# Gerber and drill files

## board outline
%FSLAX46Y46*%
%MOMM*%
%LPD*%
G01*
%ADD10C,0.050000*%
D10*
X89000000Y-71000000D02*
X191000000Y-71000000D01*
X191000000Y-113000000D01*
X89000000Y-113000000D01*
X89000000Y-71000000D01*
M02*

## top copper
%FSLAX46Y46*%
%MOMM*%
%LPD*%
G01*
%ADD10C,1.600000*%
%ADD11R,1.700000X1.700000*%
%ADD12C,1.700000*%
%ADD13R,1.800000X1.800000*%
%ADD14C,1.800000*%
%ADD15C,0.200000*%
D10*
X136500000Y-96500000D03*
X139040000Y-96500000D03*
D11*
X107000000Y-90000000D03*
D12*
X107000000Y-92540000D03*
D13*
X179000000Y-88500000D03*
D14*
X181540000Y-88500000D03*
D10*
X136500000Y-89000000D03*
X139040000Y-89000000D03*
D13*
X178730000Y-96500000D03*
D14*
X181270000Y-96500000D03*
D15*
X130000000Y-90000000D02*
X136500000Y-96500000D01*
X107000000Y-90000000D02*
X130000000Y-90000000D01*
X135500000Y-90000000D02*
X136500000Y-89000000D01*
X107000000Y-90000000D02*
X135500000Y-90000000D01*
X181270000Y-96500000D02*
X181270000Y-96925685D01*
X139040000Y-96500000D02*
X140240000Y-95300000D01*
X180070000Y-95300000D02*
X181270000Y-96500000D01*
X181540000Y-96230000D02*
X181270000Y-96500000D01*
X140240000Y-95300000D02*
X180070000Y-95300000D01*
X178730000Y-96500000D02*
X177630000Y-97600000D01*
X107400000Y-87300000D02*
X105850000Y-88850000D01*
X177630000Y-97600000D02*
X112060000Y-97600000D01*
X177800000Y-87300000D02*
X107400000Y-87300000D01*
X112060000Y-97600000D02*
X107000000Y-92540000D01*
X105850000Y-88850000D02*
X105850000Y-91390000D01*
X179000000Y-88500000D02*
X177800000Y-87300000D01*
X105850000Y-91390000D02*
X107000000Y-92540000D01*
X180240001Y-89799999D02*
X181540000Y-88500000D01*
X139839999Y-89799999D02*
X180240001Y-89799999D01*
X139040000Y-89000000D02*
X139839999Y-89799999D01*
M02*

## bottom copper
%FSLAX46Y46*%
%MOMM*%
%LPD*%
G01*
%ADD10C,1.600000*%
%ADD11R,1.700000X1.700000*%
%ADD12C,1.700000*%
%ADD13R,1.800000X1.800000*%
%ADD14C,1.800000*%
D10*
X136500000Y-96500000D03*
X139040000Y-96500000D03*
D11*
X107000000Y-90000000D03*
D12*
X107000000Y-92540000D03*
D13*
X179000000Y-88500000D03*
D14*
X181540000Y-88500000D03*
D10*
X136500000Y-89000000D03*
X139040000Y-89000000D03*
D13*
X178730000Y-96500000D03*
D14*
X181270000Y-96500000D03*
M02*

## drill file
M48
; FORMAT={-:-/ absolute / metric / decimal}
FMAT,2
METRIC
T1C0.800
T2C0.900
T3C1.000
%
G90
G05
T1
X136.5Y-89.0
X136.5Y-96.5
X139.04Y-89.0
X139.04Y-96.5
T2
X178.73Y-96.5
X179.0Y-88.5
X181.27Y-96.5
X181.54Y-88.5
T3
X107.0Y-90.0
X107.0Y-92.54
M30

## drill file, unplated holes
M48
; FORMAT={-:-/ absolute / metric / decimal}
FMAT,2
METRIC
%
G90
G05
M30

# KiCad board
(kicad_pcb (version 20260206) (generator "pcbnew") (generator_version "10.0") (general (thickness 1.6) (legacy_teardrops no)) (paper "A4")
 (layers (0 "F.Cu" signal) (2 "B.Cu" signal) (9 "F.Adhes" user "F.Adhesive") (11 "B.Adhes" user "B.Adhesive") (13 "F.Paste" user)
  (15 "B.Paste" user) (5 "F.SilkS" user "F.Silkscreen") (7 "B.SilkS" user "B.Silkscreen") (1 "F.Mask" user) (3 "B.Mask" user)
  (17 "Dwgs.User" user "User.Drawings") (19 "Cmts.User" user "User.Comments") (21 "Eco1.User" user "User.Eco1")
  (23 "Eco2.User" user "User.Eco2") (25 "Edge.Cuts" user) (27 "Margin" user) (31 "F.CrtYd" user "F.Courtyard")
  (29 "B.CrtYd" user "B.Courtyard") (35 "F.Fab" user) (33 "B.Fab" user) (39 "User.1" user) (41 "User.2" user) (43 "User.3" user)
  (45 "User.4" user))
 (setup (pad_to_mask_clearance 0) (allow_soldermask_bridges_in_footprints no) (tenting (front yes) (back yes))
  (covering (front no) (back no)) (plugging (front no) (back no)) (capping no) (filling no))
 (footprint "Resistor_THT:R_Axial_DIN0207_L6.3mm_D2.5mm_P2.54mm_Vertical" (layer "F.Cu") (at 136.5 96.5)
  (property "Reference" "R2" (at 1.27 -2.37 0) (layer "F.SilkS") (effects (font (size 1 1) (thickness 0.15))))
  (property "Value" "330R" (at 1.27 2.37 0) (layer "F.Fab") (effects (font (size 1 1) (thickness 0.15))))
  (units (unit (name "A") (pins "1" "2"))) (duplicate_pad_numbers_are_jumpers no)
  (pad "1" thru_hole circle (at 0 0) (size 1.6 1.6) (drill 0.8) (layers "*.Cu" "*.Mask") (remove_unused_layers no) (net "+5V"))
  (pad "2" thru_hole circle (at 2.54 0) (size 1.6 1.6) (drill 0.8) (layers "*.Cu" "*.Mask") (remove_unused_layers no) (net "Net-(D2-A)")))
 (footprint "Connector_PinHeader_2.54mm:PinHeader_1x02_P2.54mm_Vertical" (layer "F.Cu") (at 107 90)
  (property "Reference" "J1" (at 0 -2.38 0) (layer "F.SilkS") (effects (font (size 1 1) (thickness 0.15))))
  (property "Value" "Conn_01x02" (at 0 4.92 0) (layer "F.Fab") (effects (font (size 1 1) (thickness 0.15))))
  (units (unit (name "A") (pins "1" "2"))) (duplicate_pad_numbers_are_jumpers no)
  (pad "1" thru_hole rect (at 0 0) (size 1.7 1.7) (drill 1) (layers "*.Cu" "*.Mask") (remove_unused_layers no) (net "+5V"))
  (pad "2" thru_hole circle (at 0 2.54) (size 1.7 1.7) (drill 1) (layers "*.Cu" "*.Mask") (remove_unused_layers no) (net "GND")))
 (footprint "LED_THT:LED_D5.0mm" (layer "F.Cu") (at 179 88.5)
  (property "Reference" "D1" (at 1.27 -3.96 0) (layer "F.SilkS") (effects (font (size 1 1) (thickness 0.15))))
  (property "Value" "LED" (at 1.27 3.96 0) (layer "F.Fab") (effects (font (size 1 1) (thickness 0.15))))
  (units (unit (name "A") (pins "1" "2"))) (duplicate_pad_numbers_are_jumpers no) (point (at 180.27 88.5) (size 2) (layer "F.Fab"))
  (pad "1" thru_hole rect (at 0 0) (size 1.8 1.8) (drill 0.9) (layers "*.Cu" "*.Mask") (remove_unused_layers no) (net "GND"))
  (pad "2" thru_hole circle (at 2.54 0) (size 1.8 1.8) (drill 0.9) (layers "*.Cu" "*.Mask") (remove_unused_layers no) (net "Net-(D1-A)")))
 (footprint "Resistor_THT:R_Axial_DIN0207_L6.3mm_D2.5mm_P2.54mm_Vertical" (layer "F.Cu") (at 136.5 89)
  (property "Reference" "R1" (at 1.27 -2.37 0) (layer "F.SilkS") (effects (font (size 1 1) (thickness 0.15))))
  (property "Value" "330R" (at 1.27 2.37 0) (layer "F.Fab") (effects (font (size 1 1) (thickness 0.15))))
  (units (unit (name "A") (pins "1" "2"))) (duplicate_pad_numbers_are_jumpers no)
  (pad "1" thru_hole circle (at 0 0) (size 1.6 1.6) (drill 0.8) (layers "*.Cu" "*.Mask") (remove_unused_layers no) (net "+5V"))
  (pad "2" thru_hole circle (at 2.54 0) (size 1.6 1.6) (drill 0.8) (layers "*.Cu" "*.Mask") (remove_unused_layers no) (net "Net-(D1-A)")))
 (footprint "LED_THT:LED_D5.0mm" (layer "F.Cu") (at 178.73 96.5)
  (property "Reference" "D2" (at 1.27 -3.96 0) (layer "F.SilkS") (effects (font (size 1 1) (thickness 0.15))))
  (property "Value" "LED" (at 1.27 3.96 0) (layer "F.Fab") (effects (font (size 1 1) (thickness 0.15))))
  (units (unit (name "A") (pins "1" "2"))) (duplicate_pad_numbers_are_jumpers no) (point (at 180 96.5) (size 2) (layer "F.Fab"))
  (pad "1" thru_hole rect (at 0 0) (size 1.8 1.8) (drill 0.9) (layers "*.Cu" "*.Mask") (remove_unused_layers no) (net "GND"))
  (pad "2" thru_hole circle (at 2.54 0) (size 1.8 1.8) (drill 0.9) (layers "*.Cu" "*.Mask") (remove_unused_layers no) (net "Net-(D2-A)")))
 (gr_rect (start 89 71) (end 191 113) (stroke (width 0.05) (type default)) (fill no) (layer "Edge.Cuts"))
 (segment (start 130 90) (end 136.5 96.5) (width 0.2) (layer "F.Cu") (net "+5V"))
 (segment (start 107 90) (end 130 90) (width 0.2) (layer "F.Cu") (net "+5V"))
 (segment (start 135.5 90) (end 136.5 89) (width 0.2) (layer "F.Cu") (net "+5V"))
 (segment (start 107 90) (end 135.5 90) (width 0.2) (layer "F.Cu") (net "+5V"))
 (segment (start 181.27 96.5) (end 181.27 96.925685) (width 0.2) (layer "F.Cu") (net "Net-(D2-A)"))
 (segment (start 139.04 96.5) (end 140.24 95.3) (width 0.2) (layer "F.Cu") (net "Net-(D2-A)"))
 (segment (start 180.07 95.3) (end 181.27 96.5) (width 0.2) (layer "F.Cu") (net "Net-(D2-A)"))
 (segment (start 181.54 96.23) (end 181.27 96.5) (width 0.2) (layer "F.Cu") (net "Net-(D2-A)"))
 (segment (start 140.24 95.3) (end 180.07 95.3) (width 0.2) (layer "F.Cu") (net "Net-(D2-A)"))
 (segment (start 178.73 96.5) (end 177.63 97.6) (width 0.2) (layer "F.Cu") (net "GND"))
 (segment (start 107.4 87.3) (end 105.85 88.85) (width 0.2) (layer "F.Cu") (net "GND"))
 (segment (start 177.63 97.6) (end 112.06 97.6) (width 0.2) (layer "F.Cu") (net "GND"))
 (segment (start 177.8 87.3) (end 107.4 87.3) (width 0.2) (layer "F.Cu") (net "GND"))
 (segment (start 112.06 97.6) (end 107 92.54) (width 0.2) (layer "F.Cu") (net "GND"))
 (segment (start 105.85 88.85) (end 105.85 91.39) (width 0.2) (layer "F.Cu") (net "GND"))
 (segment (start 179 88.5) (end 177.8 87.3) (width 0.2) (layer "F.Cu") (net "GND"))
 (segment (start 105.85 91.39) (end 107 92.54) (width 0.2) (layer "F.Cu") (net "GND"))
 (segment (start 180.240001 89.799999) (end 181.54 88.5) (width 0.2) (layer "F.Cu") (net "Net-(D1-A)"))
 (segment (start 139.839999 89.799999) (end 180.240001 89.799999) (width 0.2) (layer "F.Cu") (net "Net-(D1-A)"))
 (segment (start 139.04 89) (end 139.839999 89.799999) (width 0.2) (layer "F.Cu") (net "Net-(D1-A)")))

